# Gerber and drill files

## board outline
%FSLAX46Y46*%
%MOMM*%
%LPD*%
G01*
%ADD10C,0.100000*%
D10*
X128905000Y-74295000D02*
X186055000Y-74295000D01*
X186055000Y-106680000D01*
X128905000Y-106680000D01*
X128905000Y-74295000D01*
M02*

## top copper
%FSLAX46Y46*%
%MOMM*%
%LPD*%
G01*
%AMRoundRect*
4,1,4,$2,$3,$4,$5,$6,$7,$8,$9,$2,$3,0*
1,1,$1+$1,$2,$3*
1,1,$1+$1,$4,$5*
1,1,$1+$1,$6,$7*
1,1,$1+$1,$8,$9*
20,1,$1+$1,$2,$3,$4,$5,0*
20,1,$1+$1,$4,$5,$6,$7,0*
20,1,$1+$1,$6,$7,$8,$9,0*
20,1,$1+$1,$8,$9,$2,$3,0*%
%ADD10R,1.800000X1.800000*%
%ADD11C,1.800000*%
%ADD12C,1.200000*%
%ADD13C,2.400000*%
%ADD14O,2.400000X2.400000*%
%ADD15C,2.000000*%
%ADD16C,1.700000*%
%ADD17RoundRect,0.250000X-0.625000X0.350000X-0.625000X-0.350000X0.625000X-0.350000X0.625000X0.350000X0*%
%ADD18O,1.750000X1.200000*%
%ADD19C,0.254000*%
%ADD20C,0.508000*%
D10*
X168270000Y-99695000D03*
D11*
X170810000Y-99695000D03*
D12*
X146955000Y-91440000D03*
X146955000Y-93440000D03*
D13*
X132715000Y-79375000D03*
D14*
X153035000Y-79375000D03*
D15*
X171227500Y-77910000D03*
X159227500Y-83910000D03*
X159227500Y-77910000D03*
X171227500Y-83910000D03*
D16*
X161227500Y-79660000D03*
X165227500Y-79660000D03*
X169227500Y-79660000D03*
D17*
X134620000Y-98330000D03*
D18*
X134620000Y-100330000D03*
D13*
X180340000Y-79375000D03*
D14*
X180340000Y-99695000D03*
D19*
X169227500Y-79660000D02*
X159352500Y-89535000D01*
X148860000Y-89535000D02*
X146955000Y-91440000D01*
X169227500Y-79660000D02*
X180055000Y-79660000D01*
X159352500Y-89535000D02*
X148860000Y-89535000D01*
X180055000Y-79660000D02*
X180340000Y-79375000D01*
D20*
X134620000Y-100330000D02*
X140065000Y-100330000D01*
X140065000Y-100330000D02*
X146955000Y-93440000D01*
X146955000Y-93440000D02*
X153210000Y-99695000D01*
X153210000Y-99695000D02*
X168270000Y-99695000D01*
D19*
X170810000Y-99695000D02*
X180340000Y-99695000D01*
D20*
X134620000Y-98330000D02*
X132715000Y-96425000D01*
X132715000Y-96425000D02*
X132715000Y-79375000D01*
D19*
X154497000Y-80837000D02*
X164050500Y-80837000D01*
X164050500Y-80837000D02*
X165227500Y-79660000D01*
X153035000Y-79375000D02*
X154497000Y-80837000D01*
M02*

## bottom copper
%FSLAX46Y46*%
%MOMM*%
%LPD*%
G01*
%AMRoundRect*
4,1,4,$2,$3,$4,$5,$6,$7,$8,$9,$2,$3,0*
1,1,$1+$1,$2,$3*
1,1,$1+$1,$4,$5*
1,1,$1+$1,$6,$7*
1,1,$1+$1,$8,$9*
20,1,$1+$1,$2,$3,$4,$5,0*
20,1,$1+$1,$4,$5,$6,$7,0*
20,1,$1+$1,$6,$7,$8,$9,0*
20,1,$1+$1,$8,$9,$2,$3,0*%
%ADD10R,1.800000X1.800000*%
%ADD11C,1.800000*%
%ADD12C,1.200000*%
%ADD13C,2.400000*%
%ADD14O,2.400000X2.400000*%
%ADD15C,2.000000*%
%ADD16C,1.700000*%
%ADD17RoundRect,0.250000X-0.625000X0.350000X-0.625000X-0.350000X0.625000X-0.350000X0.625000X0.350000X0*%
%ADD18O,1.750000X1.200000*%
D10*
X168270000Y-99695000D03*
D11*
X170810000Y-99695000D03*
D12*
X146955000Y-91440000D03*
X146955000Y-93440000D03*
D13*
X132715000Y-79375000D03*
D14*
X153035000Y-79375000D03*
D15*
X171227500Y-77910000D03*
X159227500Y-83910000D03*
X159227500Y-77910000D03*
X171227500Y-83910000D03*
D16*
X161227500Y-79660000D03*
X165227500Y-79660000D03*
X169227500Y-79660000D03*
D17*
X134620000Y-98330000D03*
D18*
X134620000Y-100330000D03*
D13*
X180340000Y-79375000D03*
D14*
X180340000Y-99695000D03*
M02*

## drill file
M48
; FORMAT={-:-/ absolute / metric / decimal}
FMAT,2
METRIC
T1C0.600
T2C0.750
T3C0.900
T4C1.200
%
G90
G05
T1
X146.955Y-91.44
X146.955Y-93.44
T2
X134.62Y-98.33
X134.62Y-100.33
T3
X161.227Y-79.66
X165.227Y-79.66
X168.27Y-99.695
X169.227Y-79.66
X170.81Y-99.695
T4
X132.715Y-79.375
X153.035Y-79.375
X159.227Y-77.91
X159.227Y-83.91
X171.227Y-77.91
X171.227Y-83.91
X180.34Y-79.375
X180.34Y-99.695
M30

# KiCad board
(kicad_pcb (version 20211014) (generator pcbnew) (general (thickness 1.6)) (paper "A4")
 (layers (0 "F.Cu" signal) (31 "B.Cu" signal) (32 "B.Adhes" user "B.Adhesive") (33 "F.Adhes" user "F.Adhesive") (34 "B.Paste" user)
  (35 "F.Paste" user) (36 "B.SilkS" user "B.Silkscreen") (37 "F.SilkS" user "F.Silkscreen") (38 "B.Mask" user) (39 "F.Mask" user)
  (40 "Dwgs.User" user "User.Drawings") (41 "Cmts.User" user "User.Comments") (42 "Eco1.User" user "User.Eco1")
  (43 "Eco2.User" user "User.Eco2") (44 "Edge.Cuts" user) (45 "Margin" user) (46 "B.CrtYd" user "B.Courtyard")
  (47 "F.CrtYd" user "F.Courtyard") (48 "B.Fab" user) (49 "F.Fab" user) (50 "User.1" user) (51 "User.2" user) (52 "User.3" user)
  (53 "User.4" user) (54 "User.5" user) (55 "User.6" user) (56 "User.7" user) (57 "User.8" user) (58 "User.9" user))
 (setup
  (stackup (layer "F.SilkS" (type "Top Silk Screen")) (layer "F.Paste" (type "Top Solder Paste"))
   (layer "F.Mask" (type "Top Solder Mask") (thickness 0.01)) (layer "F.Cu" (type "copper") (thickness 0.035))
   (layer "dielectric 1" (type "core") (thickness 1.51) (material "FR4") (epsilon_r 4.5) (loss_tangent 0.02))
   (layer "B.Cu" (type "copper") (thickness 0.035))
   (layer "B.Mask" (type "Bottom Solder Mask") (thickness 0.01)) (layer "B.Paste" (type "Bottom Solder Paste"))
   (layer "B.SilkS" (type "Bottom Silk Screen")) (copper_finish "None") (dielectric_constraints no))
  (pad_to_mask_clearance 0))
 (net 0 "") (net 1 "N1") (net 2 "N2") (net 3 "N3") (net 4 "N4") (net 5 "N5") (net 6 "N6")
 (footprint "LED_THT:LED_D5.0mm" (layer "F.Cu") (at 168.27 99.695)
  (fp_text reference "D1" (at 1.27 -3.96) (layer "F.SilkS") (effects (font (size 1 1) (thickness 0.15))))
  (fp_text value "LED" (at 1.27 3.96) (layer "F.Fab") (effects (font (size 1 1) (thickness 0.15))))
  (pad "1" thru_hole rect (at 0 0) (size 1.8 1.8) (drill 0.9) (layers *.Cu *.Mask) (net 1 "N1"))
  (pad "2" thru_hole circle (at 2.54 0) (size 1.8 1.8) (drill 0.9) (layers *.Cu *.Mask) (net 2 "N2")))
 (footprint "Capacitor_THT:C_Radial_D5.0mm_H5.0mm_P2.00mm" (layer "F.Cu") (at 146.955 91.44 -90)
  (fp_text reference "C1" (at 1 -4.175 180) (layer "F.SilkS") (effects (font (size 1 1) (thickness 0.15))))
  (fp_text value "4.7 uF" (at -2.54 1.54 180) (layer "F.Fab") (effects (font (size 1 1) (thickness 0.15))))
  (pad "1" thru_hole circle (at 0 0 270) (size 1.2 1.2) (drill 0.6) (layers *.Cu *.Mask) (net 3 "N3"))
  (pad "2" thru_hole circle (at 2 0 270) (size 1.2 1.2) (drill 0.6) (layers *.Cu *.Mask) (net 1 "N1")))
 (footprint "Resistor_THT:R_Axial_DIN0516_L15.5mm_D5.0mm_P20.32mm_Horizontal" (layer "F.Cu") (at 132.715 79.375)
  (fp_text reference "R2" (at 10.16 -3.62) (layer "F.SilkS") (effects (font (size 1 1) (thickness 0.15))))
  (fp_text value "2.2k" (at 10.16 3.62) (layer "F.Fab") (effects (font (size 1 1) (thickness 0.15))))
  (pad "1" thru_hole circle (at 0 0) (size 2.4 2.4) (drill 1.2) (layers *.Cu *.Mask) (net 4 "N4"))
  (pad "2" thru_hole oval (at 20.32 0) (size 2.4 2.4) (drill 1.2) (layers *.Cu *.Mask) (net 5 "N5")))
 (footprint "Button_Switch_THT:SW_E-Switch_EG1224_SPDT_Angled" (layer "F.Cu") (at 161.2275 79.66)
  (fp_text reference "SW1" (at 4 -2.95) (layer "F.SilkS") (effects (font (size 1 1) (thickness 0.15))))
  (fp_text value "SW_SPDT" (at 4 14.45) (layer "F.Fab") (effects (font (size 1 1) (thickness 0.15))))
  (pad "" thru_hole circle (at 10 -1.75) (size 2 2) (drill 1.2) (layers *.Cu *.Mask))
  (pad "" thru_hole circle (at -2 4.25) (size 2 2) (drill 1.2) (layers *.Cu *.Mask))
  (pad "" thru_hole circle (at -2 -1.75) (size 2 2) (drill 1.2) (layers *.Cu *.Mask))
  (pad "" thru_hole circle (at 10 4.25) (size 2 2) (drill 1.2) (layers *.Cu *.Mask))
  (pad "1" thru_hole circle (at 0 0) (size 1.7 1.7) (drill 0.9) (layers *.Cu *.Mask) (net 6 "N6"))
  (pad "2" thru_hole circle (at 4 0) (size 1.7 1.7) (drill 0.9) (layers *.Cu *.Mask) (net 5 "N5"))
  (pad "3" thru_hole circle (at 8 0) (size 1.7 1.7) (drill 0.9) (layers *.Cu *.Mask) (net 3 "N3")))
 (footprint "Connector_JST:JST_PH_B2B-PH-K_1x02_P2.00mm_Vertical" (layer "F.Cu") (at 134.62 98.33 -90)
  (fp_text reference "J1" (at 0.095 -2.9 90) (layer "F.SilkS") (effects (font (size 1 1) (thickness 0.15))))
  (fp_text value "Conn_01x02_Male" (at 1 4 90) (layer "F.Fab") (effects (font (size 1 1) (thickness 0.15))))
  (pad "1" thru_hole roundrect (at 0 0 270) (size 1.2 1.75) (drill 0.75) (layers *.Cu *.Mask) (roundrect_rratio 0.2083333333) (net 4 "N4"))
  (pad "2" thru_hole oval (at 2 0 270) (size 1.2 1.75) (drill 0.75) (layers *.Cu *.Mask) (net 1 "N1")))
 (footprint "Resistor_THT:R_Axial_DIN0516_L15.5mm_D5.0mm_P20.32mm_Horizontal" (layer "F.Cu") (at 180.34 79.375 -90)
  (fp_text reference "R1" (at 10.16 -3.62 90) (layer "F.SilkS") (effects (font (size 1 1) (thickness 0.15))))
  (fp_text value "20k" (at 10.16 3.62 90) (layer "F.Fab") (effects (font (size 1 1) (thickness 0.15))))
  (pad "1" thru_hole circle (at 0 0 270) (size 2.4 2.4) (drill 1.2) (layers *.Cu *.Mask) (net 3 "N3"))
  (pad "2" thru_hole oval (at 20.32 0 270) (size 2.4 2.4) (drill 1.2) (layers *.Cu *.Mask) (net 2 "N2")))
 (gr_rect (start 128.905 106.68) (end 186.055 74.295) (layer "Edge.Cuts") (width 0.1) (fill none))
 (segment (start 169.2275 79.66) (end 159.3525 89.535) (width 0.254) (layer "F.Cu") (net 3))
 (segment (start 148.86 89.535) (end 146.955 91.44) (width 0.254) (layer "F.Cu") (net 3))
 (segment (start 169.2275 79.66) (end 180.055 79.66) (width 0.254) (layer "F.Cu") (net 3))
 (segment (start 159.3525 89.535) (end 148.86 89.535) (width 0.254) (layer "F.Cu") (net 3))
 (segment (start 180.055 79.66) (end 180.34 79.375) (width 0.254) (layer "F.Cu") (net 3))
 (segment (start 134.62 100.33) (end 140.065 100.33) (width 0.508) (layer "F.Cu") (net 1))
 (segment (start 140.065 100.33) (end 146.955 93.44) (width 0.508) (layer "F.Cu") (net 1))
 (segment (start 146.955 93.44) (end 153.21 99.695) (width 0.508) (layer "F.Cu") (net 1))
 (segment (start 153.21 99.695) (end 168.27 99.695) (width 0.508) (layer "F.Cu") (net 1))
 (segment (start 170.81 99.695) (end 180.34 99.695) (width 0.254) (layer "F.Cu") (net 2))
 (segment (start 134.62 98.33) (end 132.715 96.425) (width 0.508) (layer "F.Cu") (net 4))
 (segment (start 132.715 96.425) (end 132.715 79.375) (width 0.508) (layer "F.Cu") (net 4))
 (segment (start 154.497 80.837) (end 164.0505 80.837) (width 0.254) (layer "F.Cu") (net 5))
 (segment (start 164.0505 80.837) (end 165.2275 79.66) (width 0.254) (layer "F.Cu") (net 5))
 (segment (start 153.035 79.375) (end 154.497 80.837) (width 0.254) (layer "F.Cu") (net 5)))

